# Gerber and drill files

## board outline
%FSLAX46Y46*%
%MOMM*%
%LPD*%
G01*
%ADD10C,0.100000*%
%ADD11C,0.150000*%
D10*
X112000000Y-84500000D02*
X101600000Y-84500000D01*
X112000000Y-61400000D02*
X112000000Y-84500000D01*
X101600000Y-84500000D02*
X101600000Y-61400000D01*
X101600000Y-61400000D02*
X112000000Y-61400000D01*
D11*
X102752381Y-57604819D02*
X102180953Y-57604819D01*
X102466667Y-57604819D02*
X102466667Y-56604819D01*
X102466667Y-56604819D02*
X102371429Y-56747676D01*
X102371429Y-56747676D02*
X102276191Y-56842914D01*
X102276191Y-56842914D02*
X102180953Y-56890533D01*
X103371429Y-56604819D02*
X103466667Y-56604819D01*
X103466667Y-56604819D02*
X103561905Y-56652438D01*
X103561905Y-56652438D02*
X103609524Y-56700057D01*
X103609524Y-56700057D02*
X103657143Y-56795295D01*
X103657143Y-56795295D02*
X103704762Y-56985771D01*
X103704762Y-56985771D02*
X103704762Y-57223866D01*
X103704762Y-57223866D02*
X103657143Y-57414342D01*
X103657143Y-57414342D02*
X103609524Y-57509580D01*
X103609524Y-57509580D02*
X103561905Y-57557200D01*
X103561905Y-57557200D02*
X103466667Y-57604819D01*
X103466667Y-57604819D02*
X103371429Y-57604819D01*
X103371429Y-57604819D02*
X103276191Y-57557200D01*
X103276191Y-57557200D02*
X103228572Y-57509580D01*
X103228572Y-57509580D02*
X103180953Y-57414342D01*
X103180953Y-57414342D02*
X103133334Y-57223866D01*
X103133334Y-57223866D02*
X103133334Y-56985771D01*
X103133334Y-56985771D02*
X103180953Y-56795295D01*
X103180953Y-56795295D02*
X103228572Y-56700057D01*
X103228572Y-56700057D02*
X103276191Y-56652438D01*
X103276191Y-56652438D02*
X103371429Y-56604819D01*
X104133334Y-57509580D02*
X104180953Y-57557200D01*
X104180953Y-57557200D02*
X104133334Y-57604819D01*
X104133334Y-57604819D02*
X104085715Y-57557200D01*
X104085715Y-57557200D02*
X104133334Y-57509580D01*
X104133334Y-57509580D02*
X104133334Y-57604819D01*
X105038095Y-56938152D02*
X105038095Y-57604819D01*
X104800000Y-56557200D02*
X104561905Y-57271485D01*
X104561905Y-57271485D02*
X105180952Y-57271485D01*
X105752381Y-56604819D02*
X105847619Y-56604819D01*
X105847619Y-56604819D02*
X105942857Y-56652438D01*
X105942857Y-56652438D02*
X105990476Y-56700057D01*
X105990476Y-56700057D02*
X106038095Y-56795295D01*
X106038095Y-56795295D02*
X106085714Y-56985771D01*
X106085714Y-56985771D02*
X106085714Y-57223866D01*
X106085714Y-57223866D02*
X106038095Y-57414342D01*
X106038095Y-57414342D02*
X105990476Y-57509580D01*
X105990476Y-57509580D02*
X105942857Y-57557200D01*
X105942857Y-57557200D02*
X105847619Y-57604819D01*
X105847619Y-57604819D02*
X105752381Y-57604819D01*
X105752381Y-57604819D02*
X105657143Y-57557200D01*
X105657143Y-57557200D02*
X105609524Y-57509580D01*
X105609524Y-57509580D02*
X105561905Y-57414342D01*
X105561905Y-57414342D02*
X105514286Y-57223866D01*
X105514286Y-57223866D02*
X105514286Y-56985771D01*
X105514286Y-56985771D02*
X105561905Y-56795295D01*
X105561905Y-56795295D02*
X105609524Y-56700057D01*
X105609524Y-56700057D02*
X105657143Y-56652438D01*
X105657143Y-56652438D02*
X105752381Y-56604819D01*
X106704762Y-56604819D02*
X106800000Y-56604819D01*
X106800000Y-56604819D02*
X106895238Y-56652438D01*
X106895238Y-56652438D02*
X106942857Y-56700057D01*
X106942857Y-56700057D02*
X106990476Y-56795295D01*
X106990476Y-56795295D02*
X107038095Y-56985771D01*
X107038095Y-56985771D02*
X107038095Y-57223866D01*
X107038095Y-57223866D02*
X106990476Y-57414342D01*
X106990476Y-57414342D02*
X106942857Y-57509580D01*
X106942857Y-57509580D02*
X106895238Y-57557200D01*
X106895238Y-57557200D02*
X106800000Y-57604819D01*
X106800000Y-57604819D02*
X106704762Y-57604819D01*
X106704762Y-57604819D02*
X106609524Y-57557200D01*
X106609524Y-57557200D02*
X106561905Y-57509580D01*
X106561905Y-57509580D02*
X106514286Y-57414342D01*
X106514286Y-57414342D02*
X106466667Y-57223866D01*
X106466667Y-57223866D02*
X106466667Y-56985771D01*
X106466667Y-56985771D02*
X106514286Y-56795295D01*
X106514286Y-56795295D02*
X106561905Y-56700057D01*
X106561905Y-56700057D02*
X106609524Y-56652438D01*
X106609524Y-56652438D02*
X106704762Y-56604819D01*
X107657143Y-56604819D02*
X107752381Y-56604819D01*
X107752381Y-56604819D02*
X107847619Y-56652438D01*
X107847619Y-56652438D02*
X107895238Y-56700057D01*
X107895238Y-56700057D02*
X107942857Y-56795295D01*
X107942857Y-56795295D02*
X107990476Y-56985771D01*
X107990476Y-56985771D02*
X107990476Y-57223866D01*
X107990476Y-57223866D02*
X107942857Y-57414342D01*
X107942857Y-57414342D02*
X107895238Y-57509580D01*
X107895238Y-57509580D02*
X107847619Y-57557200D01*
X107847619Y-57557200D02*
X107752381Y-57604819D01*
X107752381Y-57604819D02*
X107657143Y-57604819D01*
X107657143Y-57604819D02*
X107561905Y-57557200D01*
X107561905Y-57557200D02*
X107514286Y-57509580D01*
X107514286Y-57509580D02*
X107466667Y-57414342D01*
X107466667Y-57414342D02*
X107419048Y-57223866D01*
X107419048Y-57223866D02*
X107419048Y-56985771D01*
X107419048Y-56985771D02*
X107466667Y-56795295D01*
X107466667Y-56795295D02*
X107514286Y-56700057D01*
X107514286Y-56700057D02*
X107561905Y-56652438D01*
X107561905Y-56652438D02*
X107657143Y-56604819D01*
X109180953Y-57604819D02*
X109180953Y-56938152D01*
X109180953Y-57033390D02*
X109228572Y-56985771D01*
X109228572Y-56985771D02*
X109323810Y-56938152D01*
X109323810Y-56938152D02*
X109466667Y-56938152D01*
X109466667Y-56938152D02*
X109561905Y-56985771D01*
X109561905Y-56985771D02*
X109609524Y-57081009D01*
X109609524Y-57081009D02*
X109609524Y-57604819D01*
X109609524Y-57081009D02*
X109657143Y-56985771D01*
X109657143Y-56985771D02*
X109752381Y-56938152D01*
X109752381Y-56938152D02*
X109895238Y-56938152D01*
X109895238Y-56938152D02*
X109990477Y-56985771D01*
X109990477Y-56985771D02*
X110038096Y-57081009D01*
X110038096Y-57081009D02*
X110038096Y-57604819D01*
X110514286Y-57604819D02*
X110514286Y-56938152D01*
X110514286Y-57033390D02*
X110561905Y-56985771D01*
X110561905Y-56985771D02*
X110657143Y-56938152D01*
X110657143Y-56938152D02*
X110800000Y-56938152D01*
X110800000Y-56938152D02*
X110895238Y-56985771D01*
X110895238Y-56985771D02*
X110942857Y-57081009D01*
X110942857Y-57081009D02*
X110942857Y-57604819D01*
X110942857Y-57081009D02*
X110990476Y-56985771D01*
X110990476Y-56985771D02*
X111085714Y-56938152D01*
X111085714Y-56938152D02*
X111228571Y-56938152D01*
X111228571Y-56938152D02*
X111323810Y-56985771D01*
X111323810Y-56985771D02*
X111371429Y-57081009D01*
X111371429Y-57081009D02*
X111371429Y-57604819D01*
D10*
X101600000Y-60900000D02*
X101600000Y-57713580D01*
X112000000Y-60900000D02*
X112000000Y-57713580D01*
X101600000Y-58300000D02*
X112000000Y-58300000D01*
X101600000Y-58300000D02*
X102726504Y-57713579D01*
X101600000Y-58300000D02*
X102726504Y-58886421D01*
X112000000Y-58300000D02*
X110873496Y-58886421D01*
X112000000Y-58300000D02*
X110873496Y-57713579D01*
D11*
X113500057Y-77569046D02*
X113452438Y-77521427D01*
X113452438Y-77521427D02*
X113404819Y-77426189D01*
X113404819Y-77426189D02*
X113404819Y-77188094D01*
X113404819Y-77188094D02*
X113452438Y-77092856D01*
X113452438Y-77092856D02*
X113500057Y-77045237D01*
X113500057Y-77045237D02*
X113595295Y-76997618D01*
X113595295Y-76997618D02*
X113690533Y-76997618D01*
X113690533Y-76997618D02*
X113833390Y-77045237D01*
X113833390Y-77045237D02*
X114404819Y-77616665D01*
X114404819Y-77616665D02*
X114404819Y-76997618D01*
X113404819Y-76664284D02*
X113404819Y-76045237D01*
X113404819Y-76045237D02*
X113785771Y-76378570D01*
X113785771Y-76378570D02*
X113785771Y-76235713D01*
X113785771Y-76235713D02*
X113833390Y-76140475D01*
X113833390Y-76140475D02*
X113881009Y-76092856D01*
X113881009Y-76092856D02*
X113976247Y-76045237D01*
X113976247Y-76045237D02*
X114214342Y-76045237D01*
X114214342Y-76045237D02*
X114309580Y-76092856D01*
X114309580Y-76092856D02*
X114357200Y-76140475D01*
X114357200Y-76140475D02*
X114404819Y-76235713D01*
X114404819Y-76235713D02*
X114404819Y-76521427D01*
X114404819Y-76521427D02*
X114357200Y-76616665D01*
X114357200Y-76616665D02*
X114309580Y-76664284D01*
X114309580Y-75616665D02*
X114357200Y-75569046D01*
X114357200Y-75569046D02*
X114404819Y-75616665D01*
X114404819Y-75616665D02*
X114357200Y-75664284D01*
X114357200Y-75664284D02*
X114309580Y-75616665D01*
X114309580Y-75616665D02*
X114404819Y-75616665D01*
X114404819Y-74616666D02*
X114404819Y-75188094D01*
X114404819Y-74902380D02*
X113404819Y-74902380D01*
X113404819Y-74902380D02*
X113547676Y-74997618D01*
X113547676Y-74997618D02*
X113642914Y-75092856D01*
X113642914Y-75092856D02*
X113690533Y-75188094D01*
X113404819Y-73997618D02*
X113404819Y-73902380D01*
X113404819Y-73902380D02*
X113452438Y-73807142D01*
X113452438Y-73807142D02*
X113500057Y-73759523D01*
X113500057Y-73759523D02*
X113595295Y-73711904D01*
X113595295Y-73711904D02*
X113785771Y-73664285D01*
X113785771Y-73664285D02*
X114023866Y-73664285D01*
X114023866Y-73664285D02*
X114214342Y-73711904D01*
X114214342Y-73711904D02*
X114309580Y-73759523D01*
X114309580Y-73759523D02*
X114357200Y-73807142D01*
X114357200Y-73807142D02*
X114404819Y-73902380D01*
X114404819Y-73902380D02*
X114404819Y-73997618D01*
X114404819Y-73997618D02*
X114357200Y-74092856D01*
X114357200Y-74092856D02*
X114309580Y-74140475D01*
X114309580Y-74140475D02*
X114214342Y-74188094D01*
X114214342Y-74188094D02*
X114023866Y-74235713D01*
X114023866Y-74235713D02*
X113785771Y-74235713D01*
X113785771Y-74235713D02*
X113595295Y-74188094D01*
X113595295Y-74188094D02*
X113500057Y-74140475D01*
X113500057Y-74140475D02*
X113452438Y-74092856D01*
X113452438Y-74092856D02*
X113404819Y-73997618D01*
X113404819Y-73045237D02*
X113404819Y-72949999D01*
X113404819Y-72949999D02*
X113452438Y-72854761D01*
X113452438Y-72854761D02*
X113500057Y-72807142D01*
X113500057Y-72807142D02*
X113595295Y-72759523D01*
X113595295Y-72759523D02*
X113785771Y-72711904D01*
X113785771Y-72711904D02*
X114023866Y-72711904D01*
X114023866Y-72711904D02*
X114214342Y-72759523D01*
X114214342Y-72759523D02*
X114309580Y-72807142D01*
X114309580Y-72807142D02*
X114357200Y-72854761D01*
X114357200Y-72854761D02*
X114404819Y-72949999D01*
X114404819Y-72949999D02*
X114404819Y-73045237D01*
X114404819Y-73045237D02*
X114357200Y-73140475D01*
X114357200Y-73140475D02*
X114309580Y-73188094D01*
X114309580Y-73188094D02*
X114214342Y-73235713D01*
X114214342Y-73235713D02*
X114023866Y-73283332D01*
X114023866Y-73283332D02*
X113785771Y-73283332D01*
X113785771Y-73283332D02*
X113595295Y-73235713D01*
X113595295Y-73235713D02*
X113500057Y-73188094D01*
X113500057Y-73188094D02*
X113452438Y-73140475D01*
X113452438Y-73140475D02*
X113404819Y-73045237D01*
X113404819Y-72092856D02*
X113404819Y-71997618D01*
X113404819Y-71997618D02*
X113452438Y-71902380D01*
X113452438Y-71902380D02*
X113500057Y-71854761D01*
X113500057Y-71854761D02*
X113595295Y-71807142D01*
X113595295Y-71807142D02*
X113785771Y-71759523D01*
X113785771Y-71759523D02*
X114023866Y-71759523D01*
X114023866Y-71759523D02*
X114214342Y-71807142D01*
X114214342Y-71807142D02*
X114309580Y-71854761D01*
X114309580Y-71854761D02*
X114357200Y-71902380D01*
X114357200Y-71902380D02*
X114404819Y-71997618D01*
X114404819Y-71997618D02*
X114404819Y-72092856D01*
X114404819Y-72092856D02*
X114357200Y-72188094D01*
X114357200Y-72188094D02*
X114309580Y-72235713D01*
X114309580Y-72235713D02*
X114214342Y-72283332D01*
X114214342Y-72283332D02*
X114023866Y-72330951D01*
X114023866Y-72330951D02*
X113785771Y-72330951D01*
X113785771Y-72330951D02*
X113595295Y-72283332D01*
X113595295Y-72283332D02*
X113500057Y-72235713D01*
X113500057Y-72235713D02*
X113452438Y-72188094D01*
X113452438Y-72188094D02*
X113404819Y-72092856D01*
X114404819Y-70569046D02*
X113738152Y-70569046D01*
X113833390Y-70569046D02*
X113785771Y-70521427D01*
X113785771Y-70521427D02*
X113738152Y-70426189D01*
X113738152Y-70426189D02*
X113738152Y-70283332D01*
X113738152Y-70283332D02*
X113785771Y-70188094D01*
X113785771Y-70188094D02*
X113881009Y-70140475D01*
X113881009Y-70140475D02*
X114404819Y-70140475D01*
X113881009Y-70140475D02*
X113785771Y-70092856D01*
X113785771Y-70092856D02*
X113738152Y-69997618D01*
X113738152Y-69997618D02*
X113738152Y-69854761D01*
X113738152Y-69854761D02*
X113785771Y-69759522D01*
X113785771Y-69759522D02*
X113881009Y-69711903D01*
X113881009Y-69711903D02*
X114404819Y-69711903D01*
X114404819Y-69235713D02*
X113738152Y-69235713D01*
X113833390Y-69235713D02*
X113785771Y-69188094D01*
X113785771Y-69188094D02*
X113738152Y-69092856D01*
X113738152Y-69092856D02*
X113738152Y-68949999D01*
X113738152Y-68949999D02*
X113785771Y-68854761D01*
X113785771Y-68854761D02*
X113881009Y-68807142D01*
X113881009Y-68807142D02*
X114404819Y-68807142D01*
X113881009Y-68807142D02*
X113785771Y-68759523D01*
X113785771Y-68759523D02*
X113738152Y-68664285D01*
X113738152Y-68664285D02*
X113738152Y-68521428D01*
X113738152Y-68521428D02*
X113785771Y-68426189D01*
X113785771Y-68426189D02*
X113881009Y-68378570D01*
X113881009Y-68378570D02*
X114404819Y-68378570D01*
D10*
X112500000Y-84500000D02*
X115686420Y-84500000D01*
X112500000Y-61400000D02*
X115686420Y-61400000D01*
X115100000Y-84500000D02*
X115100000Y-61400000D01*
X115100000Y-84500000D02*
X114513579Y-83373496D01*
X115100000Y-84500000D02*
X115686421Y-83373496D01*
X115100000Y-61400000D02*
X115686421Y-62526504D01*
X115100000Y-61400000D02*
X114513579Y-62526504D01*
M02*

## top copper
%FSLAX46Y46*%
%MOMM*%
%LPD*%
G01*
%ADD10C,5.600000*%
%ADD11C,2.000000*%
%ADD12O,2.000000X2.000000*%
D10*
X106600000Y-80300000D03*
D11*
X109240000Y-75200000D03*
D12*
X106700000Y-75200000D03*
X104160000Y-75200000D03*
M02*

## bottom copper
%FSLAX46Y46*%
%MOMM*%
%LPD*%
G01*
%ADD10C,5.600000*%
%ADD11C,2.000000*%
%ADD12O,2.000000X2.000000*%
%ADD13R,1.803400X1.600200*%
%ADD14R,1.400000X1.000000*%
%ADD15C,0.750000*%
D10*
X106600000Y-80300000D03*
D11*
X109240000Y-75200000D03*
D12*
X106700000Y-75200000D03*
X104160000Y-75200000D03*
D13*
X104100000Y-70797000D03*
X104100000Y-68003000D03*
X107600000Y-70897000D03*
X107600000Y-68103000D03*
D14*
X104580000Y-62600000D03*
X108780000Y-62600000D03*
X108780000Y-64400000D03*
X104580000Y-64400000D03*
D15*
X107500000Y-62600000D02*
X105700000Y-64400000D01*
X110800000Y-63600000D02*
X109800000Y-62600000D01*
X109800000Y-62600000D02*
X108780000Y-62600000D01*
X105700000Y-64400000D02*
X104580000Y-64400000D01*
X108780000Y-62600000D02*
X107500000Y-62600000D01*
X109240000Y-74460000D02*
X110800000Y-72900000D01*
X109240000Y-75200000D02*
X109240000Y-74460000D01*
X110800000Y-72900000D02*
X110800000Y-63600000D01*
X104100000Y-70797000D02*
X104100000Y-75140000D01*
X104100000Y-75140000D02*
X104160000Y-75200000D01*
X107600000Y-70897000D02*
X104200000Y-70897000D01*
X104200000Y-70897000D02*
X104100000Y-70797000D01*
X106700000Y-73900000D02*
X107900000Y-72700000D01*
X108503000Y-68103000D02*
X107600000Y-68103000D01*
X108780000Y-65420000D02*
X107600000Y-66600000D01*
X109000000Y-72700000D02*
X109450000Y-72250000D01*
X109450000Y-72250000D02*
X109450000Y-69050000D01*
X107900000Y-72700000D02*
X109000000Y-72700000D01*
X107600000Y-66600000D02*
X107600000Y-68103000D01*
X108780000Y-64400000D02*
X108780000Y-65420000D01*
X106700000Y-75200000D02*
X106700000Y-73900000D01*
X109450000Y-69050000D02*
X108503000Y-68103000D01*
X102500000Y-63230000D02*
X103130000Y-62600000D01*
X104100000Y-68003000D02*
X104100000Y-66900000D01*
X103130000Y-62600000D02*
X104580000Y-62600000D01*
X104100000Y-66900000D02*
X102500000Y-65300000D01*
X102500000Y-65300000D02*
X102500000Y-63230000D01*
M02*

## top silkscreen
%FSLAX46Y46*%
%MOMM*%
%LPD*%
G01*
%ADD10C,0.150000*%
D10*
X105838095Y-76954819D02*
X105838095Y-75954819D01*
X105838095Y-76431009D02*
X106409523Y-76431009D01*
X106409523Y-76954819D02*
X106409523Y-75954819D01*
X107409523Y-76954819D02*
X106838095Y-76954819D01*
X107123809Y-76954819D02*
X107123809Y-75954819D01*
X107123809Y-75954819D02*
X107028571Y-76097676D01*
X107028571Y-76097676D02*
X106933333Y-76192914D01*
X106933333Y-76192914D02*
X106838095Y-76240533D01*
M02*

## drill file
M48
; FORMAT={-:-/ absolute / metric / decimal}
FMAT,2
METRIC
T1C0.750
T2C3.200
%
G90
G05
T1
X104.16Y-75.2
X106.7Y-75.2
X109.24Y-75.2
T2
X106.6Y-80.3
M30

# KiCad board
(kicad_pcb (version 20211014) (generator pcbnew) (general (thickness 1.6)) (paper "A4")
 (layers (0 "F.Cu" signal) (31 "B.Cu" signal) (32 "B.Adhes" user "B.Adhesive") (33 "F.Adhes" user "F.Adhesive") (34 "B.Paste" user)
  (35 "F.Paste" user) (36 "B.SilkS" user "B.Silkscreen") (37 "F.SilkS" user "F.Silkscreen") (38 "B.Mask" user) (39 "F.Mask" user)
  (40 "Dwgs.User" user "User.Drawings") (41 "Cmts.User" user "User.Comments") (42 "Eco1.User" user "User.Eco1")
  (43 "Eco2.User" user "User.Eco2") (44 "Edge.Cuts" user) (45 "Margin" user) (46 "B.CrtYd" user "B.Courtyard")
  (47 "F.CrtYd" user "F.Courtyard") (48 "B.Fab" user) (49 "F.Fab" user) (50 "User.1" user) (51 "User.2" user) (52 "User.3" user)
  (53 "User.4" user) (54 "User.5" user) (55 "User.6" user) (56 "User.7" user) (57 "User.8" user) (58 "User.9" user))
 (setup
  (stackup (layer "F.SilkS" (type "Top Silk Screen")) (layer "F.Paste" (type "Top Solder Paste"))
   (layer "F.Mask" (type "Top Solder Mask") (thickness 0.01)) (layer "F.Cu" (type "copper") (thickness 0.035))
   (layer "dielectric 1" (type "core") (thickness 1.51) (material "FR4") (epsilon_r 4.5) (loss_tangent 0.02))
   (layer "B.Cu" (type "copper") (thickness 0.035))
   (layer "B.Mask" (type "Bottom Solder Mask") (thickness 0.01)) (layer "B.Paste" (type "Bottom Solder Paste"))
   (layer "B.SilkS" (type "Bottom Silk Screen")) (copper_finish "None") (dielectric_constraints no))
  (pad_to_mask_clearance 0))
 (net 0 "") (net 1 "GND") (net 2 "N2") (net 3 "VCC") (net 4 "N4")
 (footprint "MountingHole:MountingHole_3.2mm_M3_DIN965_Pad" (layer "F.Cu") (at 106.6 80.3)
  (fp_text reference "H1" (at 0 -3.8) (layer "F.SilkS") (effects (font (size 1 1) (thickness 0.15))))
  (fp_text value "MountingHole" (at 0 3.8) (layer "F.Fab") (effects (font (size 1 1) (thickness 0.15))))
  (pad "1" thru_hole circle (at 0 0) (size 5.6 5.6) (drill 3.2) (layers *.Cu *.Mask)))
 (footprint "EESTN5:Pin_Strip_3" (layer "B.Cu") (at 106.7 75.2 180)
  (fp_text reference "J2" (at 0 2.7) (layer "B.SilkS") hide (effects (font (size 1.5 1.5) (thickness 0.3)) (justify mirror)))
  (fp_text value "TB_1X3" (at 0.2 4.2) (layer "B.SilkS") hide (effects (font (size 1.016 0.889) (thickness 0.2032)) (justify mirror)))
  (pad "1" thru_hole circle locked (at -2.54 0 180) (size 2 2) (drill 0.75) (layers *.Cu *.Mask "B.SilkS") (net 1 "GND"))
  (pad "2" thru_hole oval locked (at 0 0 180) (size 2 2) (drill 0.75) (layers *.Cu *.Mask "B.SilkS") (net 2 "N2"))
  (pad "3" thru_hole oval locked (at 2.54 0 180) (size 2 2) (drill 0.75) (layers *.Cu *.Mask "B.SilkS") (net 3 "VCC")))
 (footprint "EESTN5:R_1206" (layer "B.Cu") (at 104.1 69.4 -90)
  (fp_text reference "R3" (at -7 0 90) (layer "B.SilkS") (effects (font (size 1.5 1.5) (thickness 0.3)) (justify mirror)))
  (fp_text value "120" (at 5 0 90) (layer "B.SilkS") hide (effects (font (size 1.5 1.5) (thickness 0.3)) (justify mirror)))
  (pad "1" smd rect locked (at 1.397 0 270) (size 1.6002 1.8034) (layers "B.Cu" "B.Paste" "B.Mask") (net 3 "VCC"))
  (pad "2" smd rect locked (at -1.397 0 270) (size 1.6002 1.8034) (layers "B.Cu" "B.Paste" "B.Mask") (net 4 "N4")))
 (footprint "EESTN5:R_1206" (layer "B.Cu") (at 107.6 69.5 -90)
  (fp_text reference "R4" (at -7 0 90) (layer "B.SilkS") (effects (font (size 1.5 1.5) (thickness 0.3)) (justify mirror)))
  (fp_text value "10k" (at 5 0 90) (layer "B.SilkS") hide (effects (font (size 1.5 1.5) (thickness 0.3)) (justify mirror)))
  (pad "1" smd rect locked (at 1.397 0 270) (size 1.6002 1.8034) (layers "B.Cu" "B.Paste" "B.Mask") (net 3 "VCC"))
  (pad "2" smd rect locked (at -1.397 0 270) (size 1.6002 1.8034) (layers "B.Cu" "B.Paste" "B.Mask") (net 2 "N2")))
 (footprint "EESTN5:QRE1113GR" (layer "B.Cu") (at 106.68 63.5 180)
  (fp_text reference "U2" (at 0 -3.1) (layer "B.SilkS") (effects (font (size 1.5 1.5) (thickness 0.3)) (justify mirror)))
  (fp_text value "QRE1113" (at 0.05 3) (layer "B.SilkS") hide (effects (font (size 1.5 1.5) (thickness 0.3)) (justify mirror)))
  (pad "1" smd rect locked (at 2.1 0.9 180) (size 1.4 1) (layers "B.Cu" "B.Paste" "B.Mask") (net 4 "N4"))
  (pad "2" smd rect locked (at -2.1 0.9 180) (size 1.4 1) (layers "B.Cu" "B.Paste" "B.Mask") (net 1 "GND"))
  (pad "3" smd rect locked (at -2.1 -0.9 180) (size 1.4 1) (layers "B.Cu" "B.Paste" "B.Mask") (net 2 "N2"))
  (pad "4" smd rect locked (at 2.1 -0.9 180) (size 1.4 1) (layers "B.Cu" "B.Paste" "B.Mask") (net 1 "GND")))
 (gr_line (start 112 84.5) (end 101.6 84.5) (layer "Edge.Cuts") (width 0.1))
 (gr_line (start 112 61.4) (end 112 84.5) (layer "Edge.Cuts") (width 0.1))
 (gr_line locked (start 101.6 84.5) (end 101.6 61.4) (layer "Edge.Cuts") (width 0.1))
 (gr_line (start 101.6 61.4) (end 112 61.4) (layer "Edge.Cuts") (width 0.1))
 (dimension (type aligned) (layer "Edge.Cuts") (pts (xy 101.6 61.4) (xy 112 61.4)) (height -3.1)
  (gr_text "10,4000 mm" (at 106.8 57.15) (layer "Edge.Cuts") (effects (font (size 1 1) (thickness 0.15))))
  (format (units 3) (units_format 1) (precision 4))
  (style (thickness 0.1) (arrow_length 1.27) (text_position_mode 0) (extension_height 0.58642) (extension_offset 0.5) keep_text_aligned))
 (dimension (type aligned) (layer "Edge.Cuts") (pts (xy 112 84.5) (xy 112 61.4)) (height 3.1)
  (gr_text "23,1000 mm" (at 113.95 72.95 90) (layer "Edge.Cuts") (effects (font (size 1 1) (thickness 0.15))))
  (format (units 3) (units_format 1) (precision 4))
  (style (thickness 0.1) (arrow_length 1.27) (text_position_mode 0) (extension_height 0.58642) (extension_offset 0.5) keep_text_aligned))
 (segment (start 107.5 62.6) (end 105.7 64.4) (width 0.75) (layer "B.Cu") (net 1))
 (segment (start 110.8 63.6) (end 109.8 62.6) (width 0.75) (layer "B.Cu") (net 1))
 (segment (start 109.8 62.6) (end 108.78 62.6) (width 0.75) (layer "B.Cu") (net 1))
 (segment (start 105.7 64.4) (end 104.58 64.4) (width 0.75) (layer "B.Cu") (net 1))
 (segment (start 108.78 62.6) (end 107.5 62.6) (width 0.75) (layer "B.Cu") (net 1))
 (segment (start 109.24 74.46) (end 110.8 72.9) (width 0.75) (layer "B.Cu") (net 1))
 (segment (start 109.24 75.2) (end 109.24 74.46) (width 0.75) (layer "B.Cu") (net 1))
 (segment (start 110.8 72.9) (end 110.8 63.6) (width 0.75) (layer "B.Cu") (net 1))
 (segment (start 104.1 70.797) (end 104.1 75.14) (width 0.75) (layer "B.Cu") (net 3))
 (segment (start 104.1 75.14) (end 104.16 75.2) (width 0.75) (layer "B.Cu") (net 3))
 (segment (start 107.6 70.897) (end 104.2 70.897) (width 0.75) (layer "B.Cu") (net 3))
 (segment (start 104.2 70.897) (end 104.1 70.797) (width 0.75) (layer "B.Cu") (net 3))
 (segment (start 106.7 73.9) (end 107.9 72.7) (width 0.75) (layer "B.Cu") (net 2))
 (segment (start 108.503 68.103) (end 107.6 68.103) (width 0.75) (layer "B.Cu") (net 2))
 (segment (start 108.78 65.42) (end 107.6 66.6) (width 0.75) (layer "B.Cu") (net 2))
 (segment (start 109 72.7) (end 109.45 72.25) (width 0.75) (layer "B.Cu") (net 2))
 (segment (start 109.45 72.25) (end 109.45 69.05) (width 0.75) (layer "B.Cu") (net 2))
 (segment (start 107.9 72.7) (end 109 72.7) (width 0.75) (layer "B.Cu") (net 2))
 (segment (start 107.6 66.6) (end 107.6 68.103) (width 0.75) (layer "B.Cu") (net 2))
 (segment (start 108.78 64.4) (end 108.78 65.42) (width 0.75) (layer "B.Cu") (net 2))
 (segment (start 106.7 75.2) (end 106.7 73.9) (width 0.75) (layer "B.Cu") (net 2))
 (segment (start 109.45 69.05) (end 108.503 68.103) (width 0.75) (layer "B.Cu") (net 2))
 (segment (start 102.5 63.23) (end 103.13 62.6) (width 0.75) (layer "B.Cu") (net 4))
 (segment (start 104.1 68.003) (end 104.1 66.9) (width 0.75) (layer "B.Cu") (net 4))
 (segment (start 103.13 62.6) (end 104.58 62.6) (width 0.75) (layer "B.Cu") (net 4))
 (segment (start 104.1 66.9) (end 102.5 65.3) (width 0.75) (layer "B.Cu") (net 4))
 (segment (start 102.5 65.3) (end 102.5 63.23) (width 0.75) (layer "B.Cu") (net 4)))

